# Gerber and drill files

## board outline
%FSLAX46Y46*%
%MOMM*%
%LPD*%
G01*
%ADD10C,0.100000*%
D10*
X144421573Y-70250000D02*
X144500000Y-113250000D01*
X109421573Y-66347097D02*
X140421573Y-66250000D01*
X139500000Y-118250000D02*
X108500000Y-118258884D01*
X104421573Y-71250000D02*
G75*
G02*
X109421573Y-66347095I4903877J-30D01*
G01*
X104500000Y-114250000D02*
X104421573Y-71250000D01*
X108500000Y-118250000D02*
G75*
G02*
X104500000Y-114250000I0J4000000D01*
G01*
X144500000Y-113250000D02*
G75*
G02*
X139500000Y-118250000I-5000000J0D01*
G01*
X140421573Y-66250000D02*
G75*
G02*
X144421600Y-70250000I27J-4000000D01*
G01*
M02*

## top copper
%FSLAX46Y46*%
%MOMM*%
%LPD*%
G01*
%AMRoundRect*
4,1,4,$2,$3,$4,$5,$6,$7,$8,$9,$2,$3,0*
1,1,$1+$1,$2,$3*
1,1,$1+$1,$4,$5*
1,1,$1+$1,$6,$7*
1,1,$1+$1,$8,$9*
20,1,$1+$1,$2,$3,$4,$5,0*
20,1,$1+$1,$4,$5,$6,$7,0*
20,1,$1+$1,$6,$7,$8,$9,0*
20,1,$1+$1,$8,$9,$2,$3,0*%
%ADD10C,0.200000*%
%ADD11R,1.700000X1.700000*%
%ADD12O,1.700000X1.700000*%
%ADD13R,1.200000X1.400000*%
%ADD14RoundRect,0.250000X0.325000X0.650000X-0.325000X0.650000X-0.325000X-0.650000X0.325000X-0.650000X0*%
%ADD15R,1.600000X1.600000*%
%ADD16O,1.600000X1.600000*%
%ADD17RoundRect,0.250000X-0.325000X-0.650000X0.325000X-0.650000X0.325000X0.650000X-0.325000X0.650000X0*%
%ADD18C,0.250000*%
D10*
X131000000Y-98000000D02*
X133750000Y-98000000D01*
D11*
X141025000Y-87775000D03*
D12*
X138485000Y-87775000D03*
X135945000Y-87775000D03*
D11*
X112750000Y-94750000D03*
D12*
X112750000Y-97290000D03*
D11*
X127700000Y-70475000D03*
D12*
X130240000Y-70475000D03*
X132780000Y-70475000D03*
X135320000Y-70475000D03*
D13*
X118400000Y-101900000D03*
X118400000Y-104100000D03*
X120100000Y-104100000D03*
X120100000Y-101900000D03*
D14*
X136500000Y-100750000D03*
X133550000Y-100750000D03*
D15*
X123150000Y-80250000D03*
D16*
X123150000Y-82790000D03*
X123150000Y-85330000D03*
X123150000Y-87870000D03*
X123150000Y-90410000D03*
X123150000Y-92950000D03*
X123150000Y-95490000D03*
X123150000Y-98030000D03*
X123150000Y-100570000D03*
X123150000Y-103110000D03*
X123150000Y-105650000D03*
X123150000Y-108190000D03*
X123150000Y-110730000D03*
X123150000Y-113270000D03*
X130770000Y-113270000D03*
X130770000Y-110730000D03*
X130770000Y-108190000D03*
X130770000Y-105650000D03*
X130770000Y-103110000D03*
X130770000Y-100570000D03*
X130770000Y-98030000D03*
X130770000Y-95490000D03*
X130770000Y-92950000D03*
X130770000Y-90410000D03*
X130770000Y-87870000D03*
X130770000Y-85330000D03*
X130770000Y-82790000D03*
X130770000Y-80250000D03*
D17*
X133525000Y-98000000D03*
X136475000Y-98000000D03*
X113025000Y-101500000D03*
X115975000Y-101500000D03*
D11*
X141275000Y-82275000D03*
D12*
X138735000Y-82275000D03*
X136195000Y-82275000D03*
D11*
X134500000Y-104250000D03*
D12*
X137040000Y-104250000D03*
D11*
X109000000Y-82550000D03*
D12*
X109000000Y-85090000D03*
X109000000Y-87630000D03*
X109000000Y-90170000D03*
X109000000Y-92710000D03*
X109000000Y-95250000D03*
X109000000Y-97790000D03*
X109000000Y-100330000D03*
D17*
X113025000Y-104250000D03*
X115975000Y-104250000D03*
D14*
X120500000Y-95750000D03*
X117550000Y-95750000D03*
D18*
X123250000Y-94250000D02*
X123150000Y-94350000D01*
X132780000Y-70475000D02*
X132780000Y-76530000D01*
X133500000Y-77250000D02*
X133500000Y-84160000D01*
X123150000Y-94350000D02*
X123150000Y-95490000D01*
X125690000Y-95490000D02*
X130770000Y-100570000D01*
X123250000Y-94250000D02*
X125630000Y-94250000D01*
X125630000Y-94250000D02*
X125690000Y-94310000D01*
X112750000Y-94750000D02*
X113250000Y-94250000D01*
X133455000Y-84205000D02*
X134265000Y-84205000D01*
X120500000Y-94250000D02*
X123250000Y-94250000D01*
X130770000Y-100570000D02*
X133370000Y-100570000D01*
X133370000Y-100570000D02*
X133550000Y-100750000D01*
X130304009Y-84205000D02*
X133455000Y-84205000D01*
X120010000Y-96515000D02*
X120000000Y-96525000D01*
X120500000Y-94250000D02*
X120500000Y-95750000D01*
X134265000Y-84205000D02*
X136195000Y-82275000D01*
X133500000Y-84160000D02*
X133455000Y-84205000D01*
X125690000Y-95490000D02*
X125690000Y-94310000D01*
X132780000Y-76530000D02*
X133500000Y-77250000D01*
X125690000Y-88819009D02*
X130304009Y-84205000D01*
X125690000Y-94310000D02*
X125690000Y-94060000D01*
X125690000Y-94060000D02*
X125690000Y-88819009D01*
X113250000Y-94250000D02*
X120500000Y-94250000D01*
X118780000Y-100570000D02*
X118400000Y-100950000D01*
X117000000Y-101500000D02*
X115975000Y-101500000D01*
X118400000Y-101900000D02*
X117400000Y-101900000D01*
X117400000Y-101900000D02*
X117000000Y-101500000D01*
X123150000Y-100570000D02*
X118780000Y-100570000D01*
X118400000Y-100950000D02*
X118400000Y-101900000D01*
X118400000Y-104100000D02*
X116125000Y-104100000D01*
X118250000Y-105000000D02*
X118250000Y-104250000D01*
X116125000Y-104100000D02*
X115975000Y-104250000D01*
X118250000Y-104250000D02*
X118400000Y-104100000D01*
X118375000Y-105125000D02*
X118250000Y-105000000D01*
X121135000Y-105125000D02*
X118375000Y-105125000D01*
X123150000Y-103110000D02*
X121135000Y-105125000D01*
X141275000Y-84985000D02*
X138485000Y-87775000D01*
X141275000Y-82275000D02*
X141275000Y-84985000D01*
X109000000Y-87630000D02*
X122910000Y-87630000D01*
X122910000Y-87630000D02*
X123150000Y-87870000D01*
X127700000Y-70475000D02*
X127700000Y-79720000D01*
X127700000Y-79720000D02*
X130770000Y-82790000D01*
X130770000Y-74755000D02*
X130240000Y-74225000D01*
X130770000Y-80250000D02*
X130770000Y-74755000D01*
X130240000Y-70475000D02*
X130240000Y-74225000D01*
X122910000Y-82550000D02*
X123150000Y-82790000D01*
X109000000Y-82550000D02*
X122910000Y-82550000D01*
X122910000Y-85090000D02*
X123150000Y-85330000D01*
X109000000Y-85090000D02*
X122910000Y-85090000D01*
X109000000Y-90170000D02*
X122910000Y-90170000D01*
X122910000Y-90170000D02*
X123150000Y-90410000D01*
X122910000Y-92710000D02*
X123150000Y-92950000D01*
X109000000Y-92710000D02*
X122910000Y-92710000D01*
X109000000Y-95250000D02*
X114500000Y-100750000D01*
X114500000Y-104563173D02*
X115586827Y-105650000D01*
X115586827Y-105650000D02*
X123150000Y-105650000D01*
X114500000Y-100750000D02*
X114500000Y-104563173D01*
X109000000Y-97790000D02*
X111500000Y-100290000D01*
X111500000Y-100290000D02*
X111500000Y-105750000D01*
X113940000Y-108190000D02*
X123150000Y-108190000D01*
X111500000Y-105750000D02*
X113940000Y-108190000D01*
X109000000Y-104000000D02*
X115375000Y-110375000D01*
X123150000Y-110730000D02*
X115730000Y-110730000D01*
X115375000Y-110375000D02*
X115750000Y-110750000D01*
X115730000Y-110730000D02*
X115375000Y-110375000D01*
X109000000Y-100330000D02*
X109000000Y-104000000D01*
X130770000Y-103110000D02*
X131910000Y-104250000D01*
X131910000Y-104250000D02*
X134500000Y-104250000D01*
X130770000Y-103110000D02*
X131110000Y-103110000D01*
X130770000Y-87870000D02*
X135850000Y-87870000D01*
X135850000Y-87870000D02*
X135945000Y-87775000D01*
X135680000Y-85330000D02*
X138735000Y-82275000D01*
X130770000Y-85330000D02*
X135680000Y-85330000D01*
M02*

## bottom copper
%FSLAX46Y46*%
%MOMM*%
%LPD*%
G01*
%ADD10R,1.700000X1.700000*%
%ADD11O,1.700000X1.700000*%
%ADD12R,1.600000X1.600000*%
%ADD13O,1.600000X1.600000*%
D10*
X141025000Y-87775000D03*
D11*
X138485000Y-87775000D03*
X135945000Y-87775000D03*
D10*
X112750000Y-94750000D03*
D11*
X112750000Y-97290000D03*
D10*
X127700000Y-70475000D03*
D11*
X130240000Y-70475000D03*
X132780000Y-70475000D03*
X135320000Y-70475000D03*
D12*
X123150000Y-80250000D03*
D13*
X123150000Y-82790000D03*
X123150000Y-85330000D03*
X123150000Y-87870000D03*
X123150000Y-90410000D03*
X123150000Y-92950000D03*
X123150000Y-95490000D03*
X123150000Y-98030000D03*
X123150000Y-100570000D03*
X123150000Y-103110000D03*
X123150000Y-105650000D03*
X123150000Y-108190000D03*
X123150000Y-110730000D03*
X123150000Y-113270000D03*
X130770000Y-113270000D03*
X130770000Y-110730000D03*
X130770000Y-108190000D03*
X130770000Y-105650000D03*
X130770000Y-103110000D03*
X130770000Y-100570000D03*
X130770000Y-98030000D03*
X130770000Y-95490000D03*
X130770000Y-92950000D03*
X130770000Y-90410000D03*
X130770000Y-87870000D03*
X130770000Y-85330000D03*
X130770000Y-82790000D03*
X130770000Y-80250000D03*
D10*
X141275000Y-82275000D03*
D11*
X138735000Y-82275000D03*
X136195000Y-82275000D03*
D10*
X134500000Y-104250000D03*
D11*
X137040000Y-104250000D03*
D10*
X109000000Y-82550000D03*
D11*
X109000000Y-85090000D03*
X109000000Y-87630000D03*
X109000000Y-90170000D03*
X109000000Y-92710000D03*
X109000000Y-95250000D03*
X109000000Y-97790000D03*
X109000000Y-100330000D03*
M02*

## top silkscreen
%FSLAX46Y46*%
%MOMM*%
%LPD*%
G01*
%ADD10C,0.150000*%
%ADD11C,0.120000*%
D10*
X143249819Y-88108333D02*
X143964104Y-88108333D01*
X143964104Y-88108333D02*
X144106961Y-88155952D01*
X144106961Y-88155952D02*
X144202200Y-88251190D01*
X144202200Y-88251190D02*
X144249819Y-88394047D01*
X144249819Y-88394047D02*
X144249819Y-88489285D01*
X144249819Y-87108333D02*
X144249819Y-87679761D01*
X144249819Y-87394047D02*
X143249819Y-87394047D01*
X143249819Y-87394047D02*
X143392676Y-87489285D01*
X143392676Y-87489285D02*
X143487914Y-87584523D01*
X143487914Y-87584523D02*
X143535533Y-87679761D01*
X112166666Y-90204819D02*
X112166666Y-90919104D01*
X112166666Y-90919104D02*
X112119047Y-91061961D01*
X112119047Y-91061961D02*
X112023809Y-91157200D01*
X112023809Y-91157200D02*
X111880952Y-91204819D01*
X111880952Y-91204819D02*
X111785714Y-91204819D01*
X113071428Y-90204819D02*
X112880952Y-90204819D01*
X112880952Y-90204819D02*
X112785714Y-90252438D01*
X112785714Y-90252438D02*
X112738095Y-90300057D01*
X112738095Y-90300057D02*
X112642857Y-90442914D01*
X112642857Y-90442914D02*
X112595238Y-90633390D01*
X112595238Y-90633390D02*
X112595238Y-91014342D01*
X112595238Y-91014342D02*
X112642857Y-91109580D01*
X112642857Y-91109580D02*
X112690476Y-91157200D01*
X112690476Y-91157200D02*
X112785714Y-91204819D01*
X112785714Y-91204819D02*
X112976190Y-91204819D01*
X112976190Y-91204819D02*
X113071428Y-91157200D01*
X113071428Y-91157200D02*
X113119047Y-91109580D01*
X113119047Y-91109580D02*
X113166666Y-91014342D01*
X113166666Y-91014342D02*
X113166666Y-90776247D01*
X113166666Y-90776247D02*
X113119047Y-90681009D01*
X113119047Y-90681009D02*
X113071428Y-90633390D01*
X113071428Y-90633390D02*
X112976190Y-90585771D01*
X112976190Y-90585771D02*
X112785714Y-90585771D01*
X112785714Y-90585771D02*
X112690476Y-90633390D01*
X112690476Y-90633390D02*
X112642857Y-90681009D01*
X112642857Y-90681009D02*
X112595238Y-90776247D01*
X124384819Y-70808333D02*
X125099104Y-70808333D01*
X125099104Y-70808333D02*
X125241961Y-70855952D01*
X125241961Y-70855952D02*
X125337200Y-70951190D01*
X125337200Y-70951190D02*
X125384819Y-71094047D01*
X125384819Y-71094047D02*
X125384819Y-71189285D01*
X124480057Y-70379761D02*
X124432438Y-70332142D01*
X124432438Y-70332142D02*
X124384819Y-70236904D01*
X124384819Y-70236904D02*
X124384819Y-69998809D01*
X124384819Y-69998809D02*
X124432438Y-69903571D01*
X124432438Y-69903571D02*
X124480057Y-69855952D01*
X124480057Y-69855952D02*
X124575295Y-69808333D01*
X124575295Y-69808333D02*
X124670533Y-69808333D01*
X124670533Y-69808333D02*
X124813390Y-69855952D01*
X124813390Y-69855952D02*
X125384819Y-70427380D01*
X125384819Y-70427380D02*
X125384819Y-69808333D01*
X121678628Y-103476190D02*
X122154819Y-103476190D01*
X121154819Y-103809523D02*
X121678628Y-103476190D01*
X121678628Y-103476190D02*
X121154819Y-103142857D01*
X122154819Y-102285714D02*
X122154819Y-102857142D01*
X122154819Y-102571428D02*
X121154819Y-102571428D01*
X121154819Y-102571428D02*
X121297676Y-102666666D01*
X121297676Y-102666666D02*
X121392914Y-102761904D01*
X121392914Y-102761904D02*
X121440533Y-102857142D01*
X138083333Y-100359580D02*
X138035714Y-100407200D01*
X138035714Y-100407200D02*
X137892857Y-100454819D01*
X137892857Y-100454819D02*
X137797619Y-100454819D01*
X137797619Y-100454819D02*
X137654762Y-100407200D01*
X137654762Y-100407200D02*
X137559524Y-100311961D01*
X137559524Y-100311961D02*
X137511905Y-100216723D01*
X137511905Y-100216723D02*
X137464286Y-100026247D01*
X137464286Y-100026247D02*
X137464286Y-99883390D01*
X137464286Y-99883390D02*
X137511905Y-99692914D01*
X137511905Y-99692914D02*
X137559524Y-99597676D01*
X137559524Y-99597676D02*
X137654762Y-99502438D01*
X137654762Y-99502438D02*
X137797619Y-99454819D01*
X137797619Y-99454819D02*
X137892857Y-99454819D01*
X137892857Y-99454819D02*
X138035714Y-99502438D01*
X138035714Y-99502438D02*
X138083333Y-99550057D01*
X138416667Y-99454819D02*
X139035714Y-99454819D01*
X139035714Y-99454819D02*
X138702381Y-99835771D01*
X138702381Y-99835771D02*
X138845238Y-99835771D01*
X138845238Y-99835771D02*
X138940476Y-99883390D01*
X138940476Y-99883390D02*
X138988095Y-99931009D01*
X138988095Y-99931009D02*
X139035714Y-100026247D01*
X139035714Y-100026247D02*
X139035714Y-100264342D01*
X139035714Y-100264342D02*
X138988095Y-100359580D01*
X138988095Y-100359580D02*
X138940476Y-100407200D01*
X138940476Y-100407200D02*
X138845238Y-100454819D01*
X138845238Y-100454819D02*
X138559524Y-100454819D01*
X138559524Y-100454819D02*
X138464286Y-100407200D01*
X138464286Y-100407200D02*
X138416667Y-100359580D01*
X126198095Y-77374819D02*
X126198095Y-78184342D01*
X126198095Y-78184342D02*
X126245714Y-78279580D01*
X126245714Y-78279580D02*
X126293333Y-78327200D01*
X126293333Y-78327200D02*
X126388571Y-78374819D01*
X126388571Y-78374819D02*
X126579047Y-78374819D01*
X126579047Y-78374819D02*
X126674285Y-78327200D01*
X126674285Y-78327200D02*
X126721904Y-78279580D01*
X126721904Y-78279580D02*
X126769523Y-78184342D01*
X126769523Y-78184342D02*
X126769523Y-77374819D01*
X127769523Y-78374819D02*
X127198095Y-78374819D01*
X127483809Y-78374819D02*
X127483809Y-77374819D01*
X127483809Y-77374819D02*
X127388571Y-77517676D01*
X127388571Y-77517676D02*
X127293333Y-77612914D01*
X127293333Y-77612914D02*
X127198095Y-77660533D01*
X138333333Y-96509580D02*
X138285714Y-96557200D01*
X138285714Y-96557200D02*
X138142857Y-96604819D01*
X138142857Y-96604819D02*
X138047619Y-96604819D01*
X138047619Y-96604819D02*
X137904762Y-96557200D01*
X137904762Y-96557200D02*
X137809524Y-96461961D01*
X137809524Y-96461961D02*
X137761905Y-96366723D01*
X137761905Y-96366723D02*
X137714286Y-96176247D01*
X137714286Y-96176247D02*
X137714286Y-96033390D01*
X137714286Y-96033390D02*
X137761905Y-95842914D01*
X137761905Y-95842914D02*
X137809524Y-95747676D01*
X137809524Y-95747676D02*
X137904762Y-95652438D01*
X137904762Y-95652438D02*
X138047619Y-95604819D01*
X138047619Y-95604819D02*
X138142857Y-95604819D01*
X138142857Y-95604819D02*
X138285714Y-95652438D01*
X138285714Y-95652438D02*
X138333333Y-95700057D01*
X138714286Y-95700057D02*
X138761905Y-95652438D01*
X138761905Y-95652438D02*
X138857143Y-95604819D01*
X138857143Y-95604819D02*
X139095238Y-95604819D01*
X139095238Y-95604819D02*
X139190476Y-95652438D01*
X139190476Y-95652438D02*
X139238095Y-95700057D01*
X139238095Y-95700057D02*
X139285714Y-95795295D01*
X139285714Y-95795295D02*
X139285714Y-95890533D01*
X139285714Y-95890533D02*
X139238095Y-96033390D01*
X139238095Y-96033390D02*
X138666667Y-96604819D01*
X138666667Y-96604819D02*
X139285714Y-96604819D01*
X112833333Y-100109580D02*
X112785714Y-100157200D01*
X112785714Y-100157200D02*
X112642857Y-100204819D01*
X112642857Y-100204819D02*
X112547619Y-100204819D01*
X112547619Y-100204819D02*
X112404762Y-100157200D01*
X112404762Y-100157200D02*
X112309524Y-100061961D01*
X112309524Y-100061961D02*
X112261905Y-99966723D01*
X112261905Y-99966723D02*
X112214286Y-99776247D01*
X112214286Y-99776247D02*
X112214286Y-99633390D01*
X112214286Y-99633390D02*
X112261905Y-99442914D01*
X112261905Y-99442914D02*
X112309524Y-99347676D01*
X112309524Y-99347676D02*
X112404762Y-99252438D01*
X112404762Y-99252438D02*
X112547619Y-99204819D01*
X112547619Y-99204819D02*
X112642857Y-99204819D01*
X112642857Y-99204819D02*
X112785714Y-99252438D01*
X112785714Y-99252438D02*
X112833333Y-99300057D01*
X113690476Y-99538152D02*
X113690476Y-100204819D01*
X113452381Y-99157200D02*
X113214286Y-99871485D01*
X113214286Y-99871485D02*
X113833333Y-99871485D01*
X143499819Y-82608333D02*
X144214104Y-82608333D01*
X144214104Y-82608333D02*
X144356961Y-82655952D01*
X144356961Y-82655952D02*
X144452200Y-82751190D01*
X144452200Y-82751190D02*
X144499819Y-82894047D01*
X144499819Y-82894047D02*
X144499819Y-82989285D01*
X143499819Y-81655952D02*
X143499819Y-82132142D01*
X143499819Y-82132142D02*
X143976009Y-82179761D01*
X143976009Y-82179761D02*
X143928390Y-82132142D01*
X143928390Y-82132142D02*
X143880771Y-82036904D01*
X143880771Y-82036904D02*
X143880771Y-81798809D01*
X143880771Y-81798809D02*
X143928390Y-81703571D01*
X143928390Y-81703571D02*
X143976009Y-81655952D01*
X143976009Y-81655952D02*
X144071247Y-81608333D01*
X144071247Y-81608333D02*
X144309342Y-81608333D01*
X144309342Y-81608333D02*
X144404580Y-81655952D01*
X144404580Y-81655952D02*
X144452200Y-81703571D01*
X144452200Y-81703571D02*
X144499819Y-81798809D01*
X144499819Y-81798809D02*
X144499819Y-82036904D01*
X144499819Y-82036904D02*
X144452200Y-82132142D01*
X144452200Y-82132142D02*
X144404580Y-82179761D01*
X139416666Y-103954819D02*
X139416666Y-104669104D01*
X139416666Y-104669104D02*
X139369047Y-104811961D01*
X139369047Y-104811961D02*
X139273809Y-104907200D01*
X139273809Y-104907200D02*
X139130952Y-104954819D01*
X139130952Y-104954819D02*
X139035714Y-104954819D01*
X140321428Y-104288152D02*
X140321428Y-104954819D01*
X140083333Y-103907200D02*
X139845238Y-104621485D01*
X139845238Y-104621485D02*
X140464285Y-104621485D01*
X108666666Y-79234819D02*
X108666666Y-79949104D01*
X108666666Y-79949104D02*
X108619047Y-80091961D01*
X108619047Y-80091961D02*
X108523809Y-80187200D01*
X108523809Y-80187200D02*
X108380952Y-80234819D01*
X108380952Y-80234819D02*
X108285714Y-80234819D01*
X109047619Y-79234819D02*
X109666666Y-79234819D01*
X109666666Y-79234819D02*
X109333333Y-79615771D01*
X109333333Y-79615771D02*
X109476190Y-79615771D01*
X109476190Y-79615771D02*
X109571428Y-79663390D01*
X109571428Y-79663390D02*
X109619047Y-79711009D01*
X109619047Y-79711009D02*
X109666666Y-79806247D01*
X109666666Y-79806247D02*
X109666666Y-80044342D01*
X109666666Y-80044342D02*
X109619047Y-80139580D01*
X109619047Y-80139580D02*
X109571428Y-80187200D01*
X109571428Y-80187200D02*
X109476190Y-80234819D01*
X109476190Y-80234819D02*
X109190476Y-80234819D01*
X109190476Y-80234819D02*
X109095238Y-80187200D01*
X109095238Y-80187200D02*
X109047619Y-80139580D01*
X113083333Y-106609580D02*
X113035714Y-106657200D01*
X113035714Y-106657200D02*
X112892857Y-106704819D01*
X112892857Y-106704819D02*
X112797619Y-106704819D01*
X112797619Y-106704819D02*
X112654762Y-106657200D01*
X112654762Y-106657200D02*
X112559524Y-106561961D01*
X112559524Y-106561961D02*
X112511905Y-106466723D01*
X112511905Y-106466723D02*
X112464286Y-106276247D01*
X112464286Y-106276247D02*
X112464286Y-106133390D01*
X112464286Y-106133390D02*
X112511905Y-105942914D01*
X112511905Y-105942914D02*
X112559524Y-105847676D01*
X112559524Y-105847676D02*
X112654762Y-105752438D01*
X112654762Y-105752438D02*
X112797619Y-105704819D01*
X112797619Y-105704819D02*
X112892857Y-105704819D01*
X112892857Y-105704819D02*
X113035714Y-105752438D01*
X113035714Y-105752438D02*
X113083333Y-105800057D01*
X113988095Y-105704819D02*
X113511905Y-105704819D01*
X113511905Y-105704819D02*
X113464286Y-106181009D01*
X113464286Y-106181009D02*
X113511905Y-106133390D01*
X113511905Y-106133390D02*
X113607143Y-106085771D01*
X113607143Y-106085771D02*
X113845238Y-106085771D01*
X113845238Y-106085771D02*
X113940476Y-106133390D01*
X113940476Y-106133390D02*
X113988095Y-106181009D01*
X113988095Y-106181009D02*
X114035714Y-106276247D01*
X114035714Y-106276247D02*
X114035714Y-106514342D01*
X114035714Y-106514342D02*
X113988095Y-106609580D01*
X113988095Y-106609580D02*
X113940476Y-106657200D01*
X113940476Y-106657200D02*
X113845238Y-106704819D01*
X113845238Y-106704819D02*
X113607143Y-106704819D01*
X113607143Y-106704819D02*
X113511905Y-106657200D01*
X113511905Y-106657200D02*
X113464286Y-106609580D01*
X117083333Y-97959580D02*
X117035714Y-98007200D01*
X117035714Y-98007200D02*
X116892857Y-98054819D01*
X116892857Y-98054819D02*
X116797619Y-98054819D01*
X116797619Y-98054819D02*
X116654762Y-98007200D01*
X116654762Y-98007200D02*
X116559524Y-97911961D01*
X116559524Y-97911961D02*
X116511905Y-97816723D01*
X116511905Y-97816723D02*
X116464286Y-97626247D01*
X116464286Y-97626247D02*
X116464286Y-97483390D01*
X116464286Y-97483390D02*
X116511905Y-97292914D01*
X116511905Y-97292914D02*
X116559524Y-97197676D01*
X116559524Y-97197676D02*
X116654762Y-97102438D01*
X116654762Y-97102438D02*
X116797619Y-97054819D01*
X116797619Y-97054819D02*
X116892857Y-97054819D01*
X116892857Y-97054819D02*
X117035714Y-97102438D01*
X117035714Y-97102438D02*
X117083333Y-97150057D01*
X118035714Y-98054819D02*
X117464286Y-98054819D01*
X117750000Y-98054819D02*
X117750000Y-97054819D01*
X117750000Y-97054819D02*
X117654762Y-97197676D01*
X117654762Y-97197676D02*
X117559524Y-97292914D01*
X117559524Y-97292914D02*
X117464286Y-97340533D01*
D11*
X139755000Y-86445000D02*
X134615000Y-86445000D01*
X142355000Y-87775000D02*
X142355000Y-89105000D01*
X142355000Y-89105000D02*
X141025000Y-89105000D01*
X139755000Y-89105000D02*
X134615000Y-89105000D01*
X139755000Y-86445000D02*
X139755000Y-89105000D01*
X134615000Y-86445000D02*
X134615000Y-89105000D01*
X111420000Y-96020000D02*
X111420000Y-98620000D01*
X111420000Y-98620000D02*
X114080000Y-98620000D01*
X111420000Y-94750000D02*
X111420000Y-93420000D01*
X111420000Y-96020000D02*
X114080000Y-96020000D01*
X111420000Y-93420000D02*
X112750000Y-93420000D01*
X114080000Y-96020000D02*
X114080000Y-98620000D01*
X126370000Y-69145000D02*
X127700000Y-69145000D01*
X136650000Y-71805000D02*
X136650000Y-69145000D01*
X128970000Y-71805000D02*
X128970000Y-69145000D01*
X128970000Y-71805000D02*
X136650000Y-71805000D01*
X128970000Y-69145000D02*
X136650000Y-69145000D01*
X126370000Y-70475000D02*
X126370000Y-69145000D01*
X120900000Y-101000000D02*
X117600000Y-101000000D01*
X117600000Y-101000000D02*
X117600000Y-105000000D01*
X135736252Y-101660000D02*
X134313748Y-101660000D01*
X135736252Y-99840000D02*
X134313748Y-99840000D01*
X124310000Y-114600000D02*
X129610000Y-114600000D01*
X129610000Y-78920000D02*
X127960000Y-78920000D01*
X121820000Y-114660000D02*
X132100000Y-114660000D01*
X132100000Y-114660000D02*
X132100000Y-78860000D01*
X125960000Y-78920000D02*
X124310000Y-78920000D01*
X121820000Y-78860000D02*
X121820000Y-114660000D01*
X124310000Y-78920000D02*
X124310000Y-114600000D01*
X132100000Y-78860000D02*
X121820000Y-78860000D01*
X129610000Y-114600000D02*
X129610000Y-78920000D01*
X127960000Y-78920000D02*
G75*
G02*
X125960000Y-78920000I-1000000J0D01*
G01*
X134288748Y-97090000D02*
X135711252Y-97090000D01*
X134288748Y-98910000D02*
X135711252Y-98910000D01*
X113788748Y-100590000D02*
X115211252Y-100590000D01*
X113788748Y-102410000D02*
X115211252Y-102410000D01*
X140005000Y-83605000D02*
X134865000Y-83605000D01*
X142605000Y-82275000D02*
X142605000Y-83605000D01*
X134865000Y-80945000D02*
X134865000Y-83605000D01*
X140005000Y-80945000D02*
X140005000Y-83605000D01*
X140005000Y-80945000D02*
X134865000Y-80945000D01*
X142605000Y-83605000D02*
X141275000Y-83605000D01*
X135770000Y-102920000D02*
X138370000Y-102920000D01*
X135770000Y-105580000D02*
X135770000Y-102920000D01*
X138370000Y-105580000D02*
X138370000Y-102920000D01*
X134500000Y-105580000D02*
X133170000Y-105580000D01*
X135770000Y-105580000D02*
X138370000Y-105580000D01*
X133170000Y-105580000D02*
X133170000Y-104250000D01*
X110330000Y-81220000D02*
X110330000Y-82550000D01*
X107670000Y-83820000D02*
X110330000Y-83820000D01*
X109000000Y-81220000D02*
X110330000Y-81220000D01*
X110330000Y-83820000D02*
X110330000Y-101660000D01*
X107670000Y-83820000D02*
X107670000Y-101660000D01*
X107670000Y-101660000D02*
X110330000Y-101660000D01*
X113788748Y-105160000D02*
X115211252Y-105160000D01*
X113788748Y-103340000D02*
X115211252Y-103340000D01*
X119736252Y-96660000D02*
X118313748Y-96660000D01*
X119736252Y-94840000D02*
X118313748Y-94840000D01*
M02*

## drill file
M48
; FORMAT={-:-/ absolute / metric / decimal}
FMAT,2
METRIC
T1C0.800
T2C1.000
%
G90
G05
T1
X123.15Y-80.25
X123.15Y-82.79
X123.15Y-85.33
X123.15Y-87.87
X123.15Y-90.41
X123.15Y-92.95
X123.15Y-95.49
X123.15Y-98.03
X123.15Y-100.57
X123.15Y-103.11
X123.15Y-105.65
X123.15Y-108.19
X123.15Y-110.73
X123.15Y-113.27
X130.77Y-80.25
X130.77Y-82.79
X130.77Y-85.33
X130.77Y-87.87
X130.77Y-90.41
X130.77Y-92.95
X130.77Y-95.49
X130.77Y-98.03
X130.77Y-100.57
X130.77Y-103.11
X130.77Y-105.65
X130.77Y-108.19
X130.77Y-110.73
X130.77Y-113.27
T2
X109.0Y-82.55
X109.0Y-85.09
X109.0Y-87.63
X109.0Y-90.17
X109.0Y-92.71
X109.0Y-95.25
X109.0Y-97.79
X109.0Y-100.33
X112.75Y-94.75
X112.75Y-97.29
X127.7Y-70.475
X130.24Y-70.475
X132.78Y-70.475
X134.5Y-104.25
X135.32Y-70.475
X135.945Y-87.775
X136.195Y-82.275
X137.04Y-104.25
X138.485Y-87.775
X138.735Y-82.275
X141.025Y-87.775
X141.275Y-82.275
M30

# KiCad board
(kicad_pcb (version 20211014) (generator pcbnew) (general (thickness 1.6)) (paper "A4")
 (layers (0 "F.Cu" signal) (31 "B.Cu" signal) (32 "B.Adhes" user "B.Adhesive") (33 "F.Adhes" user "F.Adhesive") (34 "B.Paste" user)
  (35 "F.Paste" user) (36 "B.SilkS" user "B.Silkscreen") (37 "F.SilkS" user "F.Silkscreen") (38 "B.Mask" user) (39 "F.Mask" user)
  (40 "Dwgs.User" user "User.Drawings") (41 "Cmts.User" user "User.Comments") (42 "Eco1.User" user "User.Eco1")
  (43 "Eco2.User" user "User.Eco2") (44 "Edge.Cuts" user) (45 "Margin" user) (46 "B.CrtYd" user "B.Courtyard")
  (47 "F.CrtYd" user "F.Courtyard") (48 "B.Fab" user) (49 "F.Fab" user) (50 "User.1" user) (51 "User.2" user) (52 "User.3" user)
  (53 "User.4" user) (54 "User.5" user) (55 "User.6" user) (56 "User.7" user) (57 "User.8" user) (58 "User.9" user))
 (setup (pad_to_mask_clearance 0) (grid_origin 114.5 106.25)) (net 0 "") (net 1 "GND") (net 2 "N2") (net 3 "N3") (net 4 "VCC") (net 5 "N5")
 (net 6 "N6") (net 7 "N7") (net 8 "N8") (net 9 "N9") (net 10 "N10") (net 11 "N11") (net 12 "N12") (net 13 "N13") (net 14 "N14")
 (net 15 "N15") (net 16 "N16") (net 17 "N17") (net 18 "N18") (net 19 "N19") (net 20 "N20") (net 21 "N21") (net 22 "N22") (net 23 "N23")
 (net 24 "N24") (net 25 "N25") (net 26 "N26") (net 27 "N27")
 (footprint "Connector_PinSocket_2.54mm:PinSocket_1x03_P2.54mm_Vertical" (layer "F.Cu") (at 141.025 87.775 -90)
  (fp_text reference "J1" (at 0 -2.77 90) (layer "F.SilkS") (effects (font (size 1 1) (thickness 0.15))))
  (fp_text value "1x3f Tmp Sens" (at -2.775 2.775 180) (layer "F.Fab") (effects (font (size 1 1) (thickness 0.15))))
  (fp_line (start -1.33 1.27) (end -1.33 6.41) (layer "F.SilkS") (width 0.12))
  (fp_line (start 0 -1.33) (end 1.33 -1.33) (layer "F.SilkS") (width 0.12))
  (fp_line (start 1.33 -1.33) (end 1.33 0) (layer "F.SilkS") (width 0.12))
  (fp_line (start 1.33 1.27) (end 1.33 6.41) (layer "F.SilkS") (width 0.12))
  (fp_line (start -1.33 1.27) (end 1.33 1.27) (layer "F.SilkS") (width 0.12))
  (fp_line (start -1.33 6.41) (end 1.33 6.41) (layer "F.SilkS") (width 0.12))
  (pad "1" thru_hole rect (at 0 0 270) (size 1.7 1.7) (drill 1) (layers *.Cu *.Mask) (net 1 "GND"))
  (pad "2" thru_hole oval (at 0 2.54 270) (size 1.7 1.7) (drill 1) (layers *.Cu *.Mask) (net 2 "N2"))
  (pad "3" thru_hole oval (at 0 5.08 270) (size 1.7 1.7) (drill 1) (layers *.Cu *.Mask) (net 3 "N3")))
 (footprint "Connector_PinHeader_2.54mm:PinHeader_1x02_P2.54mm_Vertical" (layer "F.Cu") (at 112.75 94.75)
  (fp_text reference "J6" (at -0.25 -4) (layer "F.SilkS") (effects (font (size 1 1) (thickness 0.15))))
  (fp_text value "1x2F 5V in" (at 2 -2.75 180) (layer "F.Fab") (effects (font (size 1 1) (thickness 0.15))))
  (fp_line (start -1.33 1.27) (end -1.33 3.87) (layer "F.SilkS") (width 0.12))
  (fp_line (start -1.33 3.87) (end 1.33 3.87) (layer "F.SilkS") (width 0.12))
  (fp_line (start -1.33 0) (end -1.33 -1.33) (layer "F.SilkS") (width 0.12))
  (fp_line (start -1.33 1.27) (end 1.33 1.27) (layer "F.SilkS") (width 0.12))
  (fp_line (start -1.33 -1.33) (end 0 -1.33) (layer "F.SilkS") (width 0.12))
  (fp_line (start 1.33 1.27) (end 1.33 3.87) (layer "F.SilkS") (width 0.12))
  (pad "1" thru_hole rect (at 0 0) (size 1.7 1.7) (drill 1) (layers *.Cu *.Mask) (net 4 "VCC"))
  (pad "2" thru_hole oval (at 0 2.54) (size 1.7 1.7) (drill 1) (layers *.Cu *.Mask) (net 1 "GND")))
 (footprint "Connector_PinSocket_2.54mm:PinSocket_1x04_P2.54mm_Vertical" (layer "F.Cu") (at 127.7 70.475 90)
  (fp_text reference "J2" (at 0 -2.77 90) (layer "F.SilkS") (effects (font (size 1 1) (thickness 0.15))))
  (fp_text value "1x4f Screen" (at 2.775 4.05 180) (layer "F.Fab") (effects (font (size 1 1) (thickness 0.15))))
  (fp_line (start 1.33 -1.33) (end 1.33 0) (layer "F.SilkS") (width 0.12))
  (fp_line (start -1.33 8.95) (end 1.33 8.95) (layer "F.SilkS") (width 0.12))
  (fp_line (start -1.33 1.27) (end 1.33 1.27) (layer "F.SilkS") (width 0.12))
  (fp_line (start -1.33 1.27) (end -1.33 8.95) (layer "F.SilkS") (width 0.12))
  (fp_line (start 1.33 1.27) (end 1.33 8.95) (layer "F.SilkS") (width 0.12))
  (fp_line (start 0 -1.33) (end 1.33 -1.33) (layer "F.SilkS") (width 0.12))
  (pad "1" thru_hole rect (at 0 0 90) (size 1.7 1.7) (drill 1) (layers *.Cu *.Mask) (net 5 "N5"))
  (pad "2" thru_hole oval (at 0 2.54 90) (size 1.7 1.7) (drill 1) (layers *.Cu *.Mask) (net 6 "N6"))
  (pad "3" thru_hole oval (at 0 5.08 90) (size 1.7 1.7) (drill 1) (layers *.Cu *.Mask) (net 4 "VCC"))
  (pad "4" thru_hole oval (at 0 7.62 90) (size 1.7 1.7) (drill 1) (layers *.Cu *.Mask) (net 1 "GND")))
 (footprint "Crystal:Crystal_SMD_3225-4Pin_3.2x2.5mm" (layer "F.Cu") (at 119.25 103 -90)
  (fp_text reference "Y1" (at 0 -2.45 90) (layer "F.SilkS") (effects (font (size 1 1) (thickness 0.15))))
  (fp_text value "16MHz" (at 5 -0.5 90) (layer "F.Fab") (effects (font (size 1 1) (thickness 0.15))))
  (fp_line (start -2 -1.65) (end -2 1.65) (layer "F.SilkS") (width 0.12))
  (fp_line (start -2 1.65) (end 2 1.65) (layer "F.SilkS") (width 0.12))
  (pad "1" smd rect (at -1.1 0.85 270) (size 1.4 1.2) (layers "F.Cu" "F.Paste" "F.Mask") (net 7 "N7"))
  (pad "2" smd rect (at 1.1 0.85 270) (size 1.4 1.2) (layers "F.Cu" "F.Paste" "F.Mask") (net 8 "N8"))
  (pad "3" smd rect (at 1.1 -0.85 270) (size 1.4 1.2) (layers "F.Cu" "F.Paste" "F.Mask"))
  (pad "4" smd rect (at -1.1 -0.85 270) (size 1.4 1.2) (layers "F.Cu" "F.Paste" "F.Mask")))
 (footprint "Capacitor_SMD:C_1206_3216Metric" (layer "F.Cu") (at 135.025 100.75 180)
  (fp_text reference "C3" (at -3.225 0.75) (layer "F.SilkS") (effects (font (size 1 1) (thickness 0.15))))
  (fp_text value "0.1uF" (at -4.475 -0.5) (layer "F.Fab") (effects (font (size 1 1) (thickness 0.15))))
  (fp_line (start -0.711252 -0.91) (end 0.711252 -0.91) (layer "F.SilkS") (width 0.12))
  (fp_line (start -0.711252 0.91) (end 0.711252 0.91) (layer "F.SilkS") (width 0.12))
  (pad "1" smd roundrect (at -1.475 0 180) (size 1.15 1.8) (layers "F.Cu" "F.Paste" "F.Mask") (roundrect_rratio 0.217391) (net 1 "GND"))
  (pad "2" smd roundrect (at 1.475 0 180) (size 1.15 1.8) (layers "F.Cu" "F.Paste" "F.Mask") (roundrect_rratio 0.217391) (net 4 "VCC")))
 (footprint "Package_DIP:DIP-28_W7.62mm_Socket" (layer "F.Cu") (at 123.15 80.25)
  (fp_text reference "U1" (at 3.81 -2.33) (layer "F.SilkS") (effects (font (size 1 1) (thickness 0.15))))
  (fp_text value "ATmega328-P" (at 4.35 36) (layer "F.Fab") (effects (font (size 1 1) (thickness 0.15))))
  (fp_line (start 1.16 34.35) (end 6.46 34.35) (layer "F.SilkS") (width 0.12))
  (fp_line (start 6.46 -1.33) (end 4.81 -1.33) (layer "F.SilkS") (width 0.12))
  (fp_line (start -1.33 34.41) (end 8.95 34.41) (layer "F.SilkS") (width 0.12))
  (fp_line (start 8.95 34.41) (end 8.95 -1.39) (layer "F.SilkS") (width 0.12))
  (fp_line (start 2.81 -1.33) (end 1.16 -1.33) (layer "F.SilkS") (width 0.12))
  (fp_line (start -1.33 -1.39) (end -1.33 34.41) (layer "F.SilkS") (width 0.12))
  (fp_line (start 1.16 -1.33) (end 1.16 34.35) (layer "F.SilkS") (width 0.12))
  (fp_line (start 8.95 -1.39) (end -1.33 -1.39) (layer "F.SilkS") (width 0.12))
  (fp_line (start 6.46 34.35) (end 6.46 -1.33) (layer "F.SilkS") (width 0.12))
  (fp_arc (start 4.81 -1.33) (mid 3.81 -0.33) (end 2.81 -1.33) (layer "F.SilkS") (width 0.12))
  (pad "1" thru_hole rect (at 0 0) (size 1.6 1.6) (drill 0.8) (layers *.Cu *.Mask) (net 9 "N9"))
  (pad "2" thru_hole oval (at 0 2.54) (size 1.6 1.6) (drill 0.8) (layers *.Cu *.Mask) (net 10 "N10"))
  (pad "3" thru_hole oval (at 0 5.08) (size 1.6 1.6) (drill 0.8) (layers *.Cu *.Mask) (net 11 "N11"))
  (pad "4" thru_hole oval (at 0 7.62) (size 1.6 1.6) (drill 0.8) (layers *.Cu *.Mask) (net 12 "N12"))
  (pad "5" thru_hole oval (at 0 10.16) (size 1.6 1.6) (drill 0.8) (layers *.Cu *.Mask) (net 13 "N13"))
  (pad "6" thru_hole oval (at 0 12.7) (size 1.6 1.6) (drill 0.8) (layers *.Cu *.Mask) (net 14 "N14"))
  (pad "7" thru_hole oval (at 0 15.24) (size 1.6 1.6) (drill 0.8) (layers *.Cu *.Mask) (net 4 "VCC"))
  (pad "8" thru_hole oval (at 0 17.78) (size 1.6 1.6) (drill 0.8) (layers *.Cu *.Mask) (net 1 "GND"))
  (pad "9" thru_hole oval (at 0 20.32) (size 1.6 1.6) (drill 0.8) (layers *.Cu *.Mask) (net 7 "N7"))
  (pad "10" thru_hole oval (at 0 22.86) (size 1.6 1.6) (drill 0.8) (layers *.Cu *.Mask) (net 8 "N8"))
  (pad "11" thru_hole oval (at 0 25.4) (size 1.6 1.6) (drill 0.8) (layers *.Cu *.Mask) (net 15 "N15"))
  (pad "12" thru_hole oval (at 0 27.94) (size 1.6 1.6) (drill 0.8) (layers *.Cu *.Mask) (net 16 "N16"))
  (pad "13" thru_hole oval (at 0 30.48) (size 1.6 1.6) (drill 0.8) (layers *.Cu *.Mask) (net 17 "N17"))
  (pad "14" thru_hole oval (at 0 33.02) (size 1.6 1.6) (drill 0.8) (layers *.Cu *.Mask) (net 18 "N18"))
  (pad "15" thru_hole oval (at 7.62 33.02) (size 1.6 1.6) (drill 0.8) (layers *.Cu *.Mask) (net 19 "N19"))
  (pad "16" thru_hole oval (at 7.62 30.48) (size 1.6 1.6) (drill 0.8) (layers *.Cu *.Mask) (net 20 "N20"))
  (pad "17" thru_hole oval (at 7.62 27.94) (size 1.6 1.6) (drill 0.8) (layers *.Cu *.Mask) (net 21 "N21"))
  (pad "18" thru_hole oval (at 7.62 25.4) (size 1.6 1.6) (drill 0.8) (layers *.Cu *.Mask) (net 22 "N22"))
  (pad "19" thru_hole oval (at 7.62 22.86) (size 1.6 1.6) (drill 0.8) (layers *.Cu *.Mask) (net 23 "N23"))
  (pad "20" thru_hole oval (at 7.62 20.32) (size 1.6 1.6) (drill 0.8) (layers *.Cu *.Mask) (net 4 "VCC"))
  (pad "21" thru_hole oval (at 7.62 17.78) (size 1.6 1.6) (drill 0.8) (layers *.Cu *.Mask) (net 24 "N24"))
  (pad "22" thru_hole oval (at 7.62 15.24) (size 1.6 1.6) (drill 0.8) (layers *.Cu *.Mask) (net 1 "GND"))
  (pad "23" thru_hole oval (at 7.62 12.7) (size 1.6 1.6) (drill 0.8) (layers *.Cu *.Mask) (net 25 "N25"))
  (pad "24" thru_hole oval (at 7.62 10.16) (size 1.6 1.6) (drill 0.8) (layers *.Cu *.Mask) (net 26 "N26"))
  (pad "25" thru_hole oval (at 7.62 7.62) (size 1.6 1.6) (drill 0.8) (layers *.Cu *.Mask) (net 3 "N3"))
  (pad "26" thru_hole oval (at 7.62 5.08) (size 1.6 1.6) (drill 0.8) (layers *.Cu *.Mask) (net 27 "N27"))
  (pad "27" thru_hole oval (at 7.62 2.54) (size 1.6 1.6) (drill 0.8) (layers *.Cu *.Mask) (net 5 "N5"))
  (pad "28" thru_hole oval (at 7.62 0) (size 1.6 1.6) (drill 0.8) (layers *.Cu *.Mask) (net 6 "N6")))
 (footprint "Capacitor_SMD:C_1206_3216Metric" (layer "F.Cu") (at 135 98)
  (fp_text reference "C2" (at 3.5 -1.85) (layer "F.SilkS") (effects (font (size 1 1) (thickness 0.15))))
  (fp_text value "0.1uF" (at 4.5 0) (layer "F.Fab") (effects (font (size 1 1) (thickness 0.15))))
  (fp_line (start -0.711252 -0.91) (end 0.711252 -0.91) (layer "F.SilkS") (width 0.12))
  (fp_line (start -0.711252 0.91) (end 0.711252 0.91) (layer "F.SilkS") (width 0.12))
  (pad "1" smd roundrect (at -1.475 0) (size 1.15 1.8) (layers "F.Cu" "F.Paste" "F.Mask") (roundrect_rratio 0.217391) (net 24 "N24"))
  (pad "2" smd roundrect (at 1.475 0) (size 1.15 1.8) (layers "F.Cu" "F.Paste" "F.Mask") (roundrect_rratio 0.217391) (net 1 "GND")))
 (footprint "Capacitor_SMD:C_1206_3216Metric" (layer "F.Cu") (at 114.5 101.5)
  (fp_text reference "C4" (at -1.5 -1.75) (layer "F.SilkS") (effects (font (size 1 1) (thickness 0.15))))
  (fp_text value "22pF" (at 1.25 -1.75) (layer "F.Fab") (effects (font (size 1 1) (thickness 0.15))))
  (fp_line (start -0.711252 -0.91) (end 0.711252 -0.91) (layer "F.SilkS") (width 0.12))
  (fp_line (start -0.711252 0.91) (end 0.711252 0.91) (layer "F.SilkS") (width 0.12))
  (pad "1" smd roundrect (at -1.475 0) (size 1.15 1.8) (layers "F.Cu" "F.Paste" "F.Mask") (roundrect_rratio 0.217391) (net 1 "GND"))
  (pad "2" smd roundrect (at 1.475 0) (size 1.15 1.8) (layers "F.Cu" "F.Paste" "F.Mask") (roundrect_rratio 0.217391) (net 7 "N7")))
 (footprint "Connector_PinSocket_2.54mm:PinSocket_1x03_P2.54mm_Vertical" (layer "F.Cu") (at 141.275 82.275 -90)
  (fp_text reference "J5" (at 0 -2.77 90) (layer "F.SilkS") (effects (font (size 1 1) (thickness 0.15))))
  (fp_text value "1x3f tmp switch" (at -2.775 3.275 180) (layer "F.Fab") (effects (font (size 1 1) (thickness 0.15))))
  (fp_line (start 1.33 1.27) (end 1.33 6.41) (layer "F.SilkS") (width 0.12))
  (fp_line (start 0 -1.33) (end 1.33 -1.33) (layer "F.SilkS") (width 0.12))
  (fp_line (start -1.33 6.41) (end 1.33 6.41) (layer "F.SilkS") (width 0.12))
  (fp_line (start -1.33 1.27) (end 1.33 1.27) (layer "F.SilkS") (width 0.12))
  (fp_line (start -1.33 1.27) (end -1.33 6.41) (layer "F.SilkS") (width 0.12))
  (fp_line (start 1.33 -1.33) (end 1.33 0) (layer "F.SilkS") (width 0.12))
  (pad "1" thru_hole rect (at 0 0 270) (size 1.7 1.7) (drill 1) (layers *.Cu *.Mask) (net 2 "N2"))
  (pad "2" thru_hole oval (at 0 2.54 270) (size 1.7 1.7) (drill 1) (layers *.Cu *.Mask) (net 27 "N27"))
  (pad "3" thru_hole oval (at 0 5.08 270) (size 1.7 1.7) (drill 1) (layers *.Cu *.Mask) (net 4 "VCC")))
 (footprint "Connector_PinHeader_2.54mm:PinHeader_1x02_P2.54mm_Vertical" (layer "F.Cu") (at 134.5 104.25 90)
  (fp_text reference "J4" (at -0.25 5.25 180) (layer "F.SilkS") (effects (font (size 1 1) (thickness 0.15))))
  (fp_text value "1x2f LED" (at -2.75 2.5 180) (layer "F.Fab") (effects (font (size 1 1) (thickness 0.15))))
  (fp_line (start 1.33 1.27) (end 1.33 3.87) (layer "F.SilkS") (width 0.12))
  (fp_line (start -1.33 1.27) (end 1.33 1.27) (layer "F.SilkS") (width 0.12))
  (fp_line (start -1.33 3.87) (end 1.33 3.87) (layer "F.SilkS") (width 0.12))
  (fp_line (start -1.33 0) (end -1.33 -1.33) (layer "F.SilkS") (width 0.12))
  (fp_line (start -1.33 1.27) (end -1.33 3.87) (layer "F.SilkS") (width 0.12))
  (fp_line (start -1.33 -1.33) (end 0 -1.33) (layer "F.SilkS") (width 0.12))
  (pad "1" thru_hole rect (at 0 0 90) (size 1.7 1.7) (drill 1) (layers *.Cu *.Mask) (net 23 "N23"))
  (pad "2" thru_hole oval (at 0 2.54 90) (size 1.7 1.7) (drill 1) (layers *.Cu *.Mask) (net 1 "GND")))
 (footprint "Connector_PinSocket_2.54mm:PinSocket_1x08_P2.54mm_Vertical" (layer "F.Cu") (at 109 82.55)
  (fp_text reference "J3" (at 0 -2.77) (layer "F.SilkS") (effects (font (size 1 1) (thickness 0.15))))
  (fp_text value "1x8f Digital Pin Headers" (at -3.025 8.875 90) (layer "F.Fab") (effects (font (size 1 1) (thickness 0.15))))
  (fp_line (start 1.33 -1.33) (end 1.33 0) (layer "F.SilkS") (width 0.12))
  (fp_line (start -1.33 1.27) (end 1.33 1.27) (layer "F.SilkS") (width 0.12))
  (fp_line (start 0 -1.33) (end 1.33 -1.33) (layer "F.SilkS") (width 0.12))
  (fp_line (start 1.33 1.27) (end 1.33 19.11) (layer "F.SilkS") (width 0.12))
  (fp_line (start -1.33 1.27) (end -1.33 19.11) (layer "F.SilkS") (width 0.12))
  (fp_line (start -1.33 19.11) (end 1.33 19.11) (layer "F.SilkS") (width 0.12))
  (pad "1" thru_hole rect (at 0 0) (size 1.7 1.7) (drill 1) (layers *.Cu *.Mask) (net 10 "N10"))
  (pad "2" thru_hole oval (at 0 2.54) (size 1.7 1.7) (drill 1) (layers *.Cu *.Mask) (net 11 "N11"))
  (pad "3" thru_hole oval (at 0 5.08) (size 1.7 1.7) (drill 1) (layers *.Cu *.Mask) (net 12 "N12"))
  (pad "4" thru_hole oval (at 0 7.62) (size 1.7 1.7) (drill 1) (layers *.Cu *.Mask) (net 13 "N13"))
  (pad "5" thru_hole oval (at 0 10.16) (size 1.7 1.7) (drill 1) (layers *.Cu *.Mask) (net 14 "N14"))
  (pad "6" thru_hole oval (at 0 12.7) (size 1.7 1.7) (drill 1) (layers *.Cu *.Mask) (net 15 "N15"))
  (pad "7" thru_hole oval (at 0 15.24) (size 1.7 1.7) (drill 1) (layers *.Cu *.Mask) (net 16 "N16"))
  (pad "8" thru_hole oval (at 0 17.78) (size 1.7 1.7) (drill 1) (layers *.Cu *.Mask) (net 17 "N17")))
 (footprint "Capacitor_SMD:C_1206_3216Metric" (layer "F.Cu") (at 114.5 104.25)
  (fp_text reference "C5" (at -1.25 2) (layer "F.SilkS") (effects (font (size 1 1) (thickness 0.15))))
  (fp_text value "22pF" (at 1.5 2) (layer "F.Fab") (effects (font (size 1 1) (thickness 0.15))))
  (fp_line (start -0.711252 0.91) (end 0.711252 0.91) (layer "F.SilkS") (width 0.12))
  (fp_line (start -0.711252 -0.91) (end 0.711252 -0.91) (layer "F.SilkS") (width 0.12))
  (pad "1" smd roundrect (at -1.475 0) (size 1.15 1.8) (layers "F.Cu" "F.Paste" "F.Mask") (roundrect_rratio 0.217391) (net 1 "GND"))
  (pad "2" smd roundrect (at 1.475 0) (size 1.15 1.8) (layers "F.Cu" "F.Paste" "F.Mask") (roundrect_rratio 0.217391) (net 8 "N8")))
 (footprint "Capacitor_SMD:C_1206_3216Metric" (layer "F.Cu") (at 119.025 95.75 180)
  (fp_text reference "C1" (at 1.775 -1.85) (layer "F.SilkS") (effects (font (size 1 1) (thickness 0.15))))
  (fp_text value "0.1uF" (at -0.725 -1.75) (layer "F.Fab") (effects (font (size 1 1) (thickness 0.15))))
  (fp_line (start -0.711252 -0.91) (end 0.711252 -0.91) (layer "F.SilkS") (width 0.12))
  (fp_line (start -0.711252 0.91) (end 0.711252 0.91) (layer "F.SilkS") (width 0.12))
  (pad "1" smd roundrect (at -1.475 0 180) (size 1.15 1.8) (layers "F.Cu" "F.Paste" "F.Mask") (roundrect_rratio 0.217391) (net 4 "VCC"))
  (pad "2" smd roundrect (at 1.475 0 180) (size 1.15 1.8) (layers "F.Cu" "F.Paste" "F.Mask") (roundrect_rratio 0.217391) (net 1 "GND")))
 (gr_line (start 131 98) (end 133.75 98) (layer "F.Cu") (width 0.2))
 (gr_line (start 144.421573 70.25) (end 144.5 113.25) (layer "Edge.Cuts") (width 0.1))
 (gr_line (start 109.421573 66.347097) (end 140.421573 66.25) (layer "Edge.Cuts") (width 0.1))
 (gr_line (start 139.5 118.25) (end 108.5 118.258884) (layer "Edge.Cuts") (width 0.1))
 (gr_arc (start 104.421573 71.25) (mid 105.892043 67.748643) (end 109.421573 66.347097) (layer "Edge.Cuts") (width 0.1))
 (gr_line (start 104.5 114.25) (end 104.421573 71.25) (layer "Edge.Cuts") (width 0.1))
 (gr_arc (start 108.5 118.25) (mid 105.671573 117.078427) (end 104.5 114.25) (layer "Edge.Cuts") (width 0.1))
 (gr_arc (start 144.5 113.25) (mid 143.035534 116.785534) (end 139.5 118.25) (layer "Edge.Cuts") (width 0.1))
 (gr_arc (start 140.421573 66.25) (mid 143.25 67.421573) (end 144.421573 70.25) (layer "Edge.Cuts") (width 0.1))
 (segment (start 123.25 94.25) (end 123.15 94.35) (width 0.25) (layer "F.Cu") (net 4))
 (segment (start 132.78 70.475) (end 132.78 76.53) (width 0.25) (layer "F.Cu") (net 4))
 (segment (start 133.5 77.25) (end 133.5 84.16) (width 0.25) (layer "F.Cu") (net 4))
 (segment (start 123.15 94.35) (end 123.15 95.49) (width 0.25) (layer "F.Cu") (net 4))
 (segment (start 125.69 95.49) (end 130.77 100.57) (width 0.25) (layer "F.Cu") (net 4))
 (segment (start 123.25 94.25) (end 125.63 94.25) (width 0.25) (layer "F.Cu") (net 4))
 (segment (start 125.63 94.25) (end 125.69 94.31) (width 0.25) (layer "F.Cu") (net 4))
 (segment (start 112.75 94.75) (end 113.25 94.25) (width 0.25) (layer "F.Cu") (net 4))
 (segment (start 133.455 84.205) (end 134.265 84.205) (width 0.25) (layer "F.Cu") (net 4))
 (segment (start 120.5 94.25) (end 123.25 94.25) (width 0.25) (layer "F.Cu") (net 4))
 (segment (start 130.77 100.57) (end 133.37 100.57) (width 0.25) (layer "F.Cu") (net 4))
 (segment (start 133.37 100.57) (end 133.55 100.75) (width 0.25) (layer "F.Cu") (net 4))
 (segment (start 130.304009 84.205) (end 133.455 84.205) (width 0.25) (layer "F.Cu") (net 4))
 (segment (start 120.01 96.515) (end 120 96.525) (width 0.25) (layer "F.Cu") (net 4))
 (segment (start 120.5 94.25) (end 120.5 95.75) (width 0.25) (layer "F.Cu") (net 4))
 (segment (start 134.265 84.205) (end 136.195 82.275) (width 0.25) (layer "F.Cu") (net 4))
 (segment (start 133.5 84.16) (end 133.455 84.205) (width 0.25) (layer "F.Cu") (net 4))
 (segment (start 125.69 95.49) (end 125.69 94.31) (width 0.25) (layer "F.Cu") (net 4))
 (segment (start 132.78 76.53) (end 133.5 77.25) (width 0.25) (layer "F.Cu") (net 4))
 (segment (start 125.69 88.819009) (end 130.304009 84.205) (width 0.25) (layer "F.Cu") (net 4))
 (segment (start 125.69 94.31) (end 125.69 94.06) (width 0.25) (layer "F.Cu") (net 4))
 (segment (start 125.69 94.06) (end 125.69 88.819009) (width 0.25) (layer "F.Cu") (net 4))
 (segment (start 113.25 94.25) (end 120.5 94.25) (width 0.25) (layer "F.Cu") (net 4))
 (segment (start 118.78 100.57) (end 118.4 100.95) (width 0.25) (layer "F.Cu") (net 7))
 (segment (start 117 101.5) (end 115.975 101.5) (width 0.25) (layer "F.Cu") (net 7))
 (segment (start 118.4 101.9) (end 117.4 101.9) (width 0.25) (layer "F.Cu") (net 7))
 (segment (start 117.4 101.9) (end 117 101.5) (width 0.25) (layer "F.Cu") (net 7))
 (segment (start 123.15 100.57) (end 118.78 100.57) (width 0.25) (layer "F.Cu") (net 7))
 (segment (start 118.4 100.95) (end 118.4 101.9) (width 0.25) (layer "F.Cu") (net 7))
 (segment (start 118.4 104.1) (end 116.125 104.1) (width 0.25) (layer "F.Cu") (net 8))
 (segment (start 118.25 105) (end 118.25 104.25) (width 0.25) (layer "F.Cu") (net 8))
 (segment (start 116.125 104.1) (end 115.975 104.25) (width 0.25) (layer "F.Cu") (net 8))
 (segment (start 118.25 104.25) (end 118.4 104.1) (width 0.25) (layer "F.Cu") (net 8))
 (segment (start 118.375 105.125) (end 118.25 105) (width 0.25) (layer "F.Cu") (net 8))
 (segment (start 121.135 105.125) (end 118.375 105.125) (width 0.25) (layer "F.Cu") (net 8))
 (segment (start 123.15 103.11) (end 121.135 105.125) (width 0.25) (layer "F.Cu") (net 8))
 (segment (start 141.275 84.985) (end 138.485 87.775) (width 0.25) (layer "F.Cu") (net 2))
 (segment (start 141.275 82.275) (end 141.275 84.985) (width 0.25) (layer "F.Cu") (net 2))
 (segment (start 109 87.63) (end 122.91 87.63) (width 0.25) (layer "F.Cu") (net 12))
 (segment (start 122.91 87.63) (end 123.15 87.87) (width 0.25) (layer "F.Cu") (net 12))
 (segment (start 127.7 70.475) (end 127.7 79.72) (width 0.25) (layer "F.Cu") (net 5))
 (segment (start 127.7 79.72) (end 130.77 82.79) (width 0.25) (layer "F.Cu") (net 5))
 (segment (start 130.77 74.755) (end 130.24 74.225) (width 0.25) (layer "F.Cu") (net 6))
 (segment (start 130.77 80.25) (end 130.77 74.755) (width 0.25) (layer "F.Cu") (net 6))
 (segment (start 130.24 70.475) (end 130.24 74.225) (width 0.25) (layer "F.Cu") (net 6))
 (segment (start 122.91 82.55) (end 123.15 82.79) (width 0.25) (layer "F.Cu") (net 10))
 (segment (start 109 82.55) (end 122.91 82.55) (width 0.25) (layer "F.Cu") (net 10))
 (segment (start 122.91 85.09) (end 123.15 85.33) (width 0.25) (layer "F.Cu") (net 11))
 (segment (start 109 85.09) (end 122.91 85.09) (width 0.25) (layer "F.Cu") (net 11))
 (segment (start 109 90.17) (end 122.91 90.17) (width 0.25) (layer "F.Cu") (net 13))
 (segment (start 122.91 90.17) (end 123.15 90.41) (width 0.25) (layer "F.Cu") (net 13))
 (segment (start 122.91 92.71) (end 123.15 92.95) (width 0.25) (layer "F.Cu") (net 14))
 (segment (start 109 92.71) (end 122.91 92.71) (width 0.25) (layer "F.Cu") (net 14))
 (segment (start 109 95.25) (end 114.5 100.75) (width 0.25) (layer "F.Cu") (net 15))
 (segment (start 114.5 104.563173) (end 115.586827 105.65) (width 0.25) (layer "F.Cu") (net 15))
 (segment (start 115.586827 105.65) (end 123.15 105.65) (width 0.25) (layer "F.Cu") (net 15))
 (segment (start 114.5 100.75) (end 114.5 104.563173) (width 0.25) (layer "F.Cu") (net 15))
 (segment (start 109 97.79) (end 111.5 100.29) (width 0.25) (layer "F.Cu") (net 16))
 (segment (start 111.5 100.29) (end 111.5 105.75) (width 0.25) (layer "F.Cu") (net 16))
 (segment (start 113.94 108.19) (end 123.15 108.19) (width 0.25) (layer "F.Cu") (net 16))
 (segment (start 111.5 105.75) (end 113.94 108.19) (width 0.25) (layer "F.Cu") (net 16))
 (segment (start 109 104) (end 115.375 110.375) (width 0.25) (layer "F.Cu") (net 17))
 (segment (start 123.15 110.73) (end 115.73 110.73) (width 0.25) (layer "F.Cu") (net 17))
 (segment (start 115.375 110.375) (end 115.75 110.75) (width 0.25) (layer "F.Cu") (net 17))
 (segment (start 115.73 110.73) (end 115.375 110.375) (width 0.25) (layer "F.Cu") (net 17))
 (segment (start 109 100.33) (end 109 104) (width 0.25) (layer "F.Cu") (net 17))
 (segment (start 130.77 103.11) (end 131.91 104.25) (width 0.25) (layer "F.Cu") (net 23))
 (segment (start 131.91 104.25) (end 134.5 104.25) (width 0.25) (layer "F.Cu") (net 23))
 (segment (start 130.77 103.11) (end 131.11 103.11) (width 0.25) (layer "F.Cu") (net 23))
 (segment (start 130.77 87.87) (end 135.85 87.87) (width 0.25) (layer "F.Cu") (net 3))
 (segment (start 135.85 87.87) (end 135.945 87.775) (width 0.25) (layer "F.Cu") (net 3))
 (segment (start 135.68 85.33) (end 138.735 82.275) (width 0.25) (layer "F.Cu") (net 27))
 (segment (start 130.77 85.33) (end 135.68 85.33) (width 0.25) (layer "F.Cu") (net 27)))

